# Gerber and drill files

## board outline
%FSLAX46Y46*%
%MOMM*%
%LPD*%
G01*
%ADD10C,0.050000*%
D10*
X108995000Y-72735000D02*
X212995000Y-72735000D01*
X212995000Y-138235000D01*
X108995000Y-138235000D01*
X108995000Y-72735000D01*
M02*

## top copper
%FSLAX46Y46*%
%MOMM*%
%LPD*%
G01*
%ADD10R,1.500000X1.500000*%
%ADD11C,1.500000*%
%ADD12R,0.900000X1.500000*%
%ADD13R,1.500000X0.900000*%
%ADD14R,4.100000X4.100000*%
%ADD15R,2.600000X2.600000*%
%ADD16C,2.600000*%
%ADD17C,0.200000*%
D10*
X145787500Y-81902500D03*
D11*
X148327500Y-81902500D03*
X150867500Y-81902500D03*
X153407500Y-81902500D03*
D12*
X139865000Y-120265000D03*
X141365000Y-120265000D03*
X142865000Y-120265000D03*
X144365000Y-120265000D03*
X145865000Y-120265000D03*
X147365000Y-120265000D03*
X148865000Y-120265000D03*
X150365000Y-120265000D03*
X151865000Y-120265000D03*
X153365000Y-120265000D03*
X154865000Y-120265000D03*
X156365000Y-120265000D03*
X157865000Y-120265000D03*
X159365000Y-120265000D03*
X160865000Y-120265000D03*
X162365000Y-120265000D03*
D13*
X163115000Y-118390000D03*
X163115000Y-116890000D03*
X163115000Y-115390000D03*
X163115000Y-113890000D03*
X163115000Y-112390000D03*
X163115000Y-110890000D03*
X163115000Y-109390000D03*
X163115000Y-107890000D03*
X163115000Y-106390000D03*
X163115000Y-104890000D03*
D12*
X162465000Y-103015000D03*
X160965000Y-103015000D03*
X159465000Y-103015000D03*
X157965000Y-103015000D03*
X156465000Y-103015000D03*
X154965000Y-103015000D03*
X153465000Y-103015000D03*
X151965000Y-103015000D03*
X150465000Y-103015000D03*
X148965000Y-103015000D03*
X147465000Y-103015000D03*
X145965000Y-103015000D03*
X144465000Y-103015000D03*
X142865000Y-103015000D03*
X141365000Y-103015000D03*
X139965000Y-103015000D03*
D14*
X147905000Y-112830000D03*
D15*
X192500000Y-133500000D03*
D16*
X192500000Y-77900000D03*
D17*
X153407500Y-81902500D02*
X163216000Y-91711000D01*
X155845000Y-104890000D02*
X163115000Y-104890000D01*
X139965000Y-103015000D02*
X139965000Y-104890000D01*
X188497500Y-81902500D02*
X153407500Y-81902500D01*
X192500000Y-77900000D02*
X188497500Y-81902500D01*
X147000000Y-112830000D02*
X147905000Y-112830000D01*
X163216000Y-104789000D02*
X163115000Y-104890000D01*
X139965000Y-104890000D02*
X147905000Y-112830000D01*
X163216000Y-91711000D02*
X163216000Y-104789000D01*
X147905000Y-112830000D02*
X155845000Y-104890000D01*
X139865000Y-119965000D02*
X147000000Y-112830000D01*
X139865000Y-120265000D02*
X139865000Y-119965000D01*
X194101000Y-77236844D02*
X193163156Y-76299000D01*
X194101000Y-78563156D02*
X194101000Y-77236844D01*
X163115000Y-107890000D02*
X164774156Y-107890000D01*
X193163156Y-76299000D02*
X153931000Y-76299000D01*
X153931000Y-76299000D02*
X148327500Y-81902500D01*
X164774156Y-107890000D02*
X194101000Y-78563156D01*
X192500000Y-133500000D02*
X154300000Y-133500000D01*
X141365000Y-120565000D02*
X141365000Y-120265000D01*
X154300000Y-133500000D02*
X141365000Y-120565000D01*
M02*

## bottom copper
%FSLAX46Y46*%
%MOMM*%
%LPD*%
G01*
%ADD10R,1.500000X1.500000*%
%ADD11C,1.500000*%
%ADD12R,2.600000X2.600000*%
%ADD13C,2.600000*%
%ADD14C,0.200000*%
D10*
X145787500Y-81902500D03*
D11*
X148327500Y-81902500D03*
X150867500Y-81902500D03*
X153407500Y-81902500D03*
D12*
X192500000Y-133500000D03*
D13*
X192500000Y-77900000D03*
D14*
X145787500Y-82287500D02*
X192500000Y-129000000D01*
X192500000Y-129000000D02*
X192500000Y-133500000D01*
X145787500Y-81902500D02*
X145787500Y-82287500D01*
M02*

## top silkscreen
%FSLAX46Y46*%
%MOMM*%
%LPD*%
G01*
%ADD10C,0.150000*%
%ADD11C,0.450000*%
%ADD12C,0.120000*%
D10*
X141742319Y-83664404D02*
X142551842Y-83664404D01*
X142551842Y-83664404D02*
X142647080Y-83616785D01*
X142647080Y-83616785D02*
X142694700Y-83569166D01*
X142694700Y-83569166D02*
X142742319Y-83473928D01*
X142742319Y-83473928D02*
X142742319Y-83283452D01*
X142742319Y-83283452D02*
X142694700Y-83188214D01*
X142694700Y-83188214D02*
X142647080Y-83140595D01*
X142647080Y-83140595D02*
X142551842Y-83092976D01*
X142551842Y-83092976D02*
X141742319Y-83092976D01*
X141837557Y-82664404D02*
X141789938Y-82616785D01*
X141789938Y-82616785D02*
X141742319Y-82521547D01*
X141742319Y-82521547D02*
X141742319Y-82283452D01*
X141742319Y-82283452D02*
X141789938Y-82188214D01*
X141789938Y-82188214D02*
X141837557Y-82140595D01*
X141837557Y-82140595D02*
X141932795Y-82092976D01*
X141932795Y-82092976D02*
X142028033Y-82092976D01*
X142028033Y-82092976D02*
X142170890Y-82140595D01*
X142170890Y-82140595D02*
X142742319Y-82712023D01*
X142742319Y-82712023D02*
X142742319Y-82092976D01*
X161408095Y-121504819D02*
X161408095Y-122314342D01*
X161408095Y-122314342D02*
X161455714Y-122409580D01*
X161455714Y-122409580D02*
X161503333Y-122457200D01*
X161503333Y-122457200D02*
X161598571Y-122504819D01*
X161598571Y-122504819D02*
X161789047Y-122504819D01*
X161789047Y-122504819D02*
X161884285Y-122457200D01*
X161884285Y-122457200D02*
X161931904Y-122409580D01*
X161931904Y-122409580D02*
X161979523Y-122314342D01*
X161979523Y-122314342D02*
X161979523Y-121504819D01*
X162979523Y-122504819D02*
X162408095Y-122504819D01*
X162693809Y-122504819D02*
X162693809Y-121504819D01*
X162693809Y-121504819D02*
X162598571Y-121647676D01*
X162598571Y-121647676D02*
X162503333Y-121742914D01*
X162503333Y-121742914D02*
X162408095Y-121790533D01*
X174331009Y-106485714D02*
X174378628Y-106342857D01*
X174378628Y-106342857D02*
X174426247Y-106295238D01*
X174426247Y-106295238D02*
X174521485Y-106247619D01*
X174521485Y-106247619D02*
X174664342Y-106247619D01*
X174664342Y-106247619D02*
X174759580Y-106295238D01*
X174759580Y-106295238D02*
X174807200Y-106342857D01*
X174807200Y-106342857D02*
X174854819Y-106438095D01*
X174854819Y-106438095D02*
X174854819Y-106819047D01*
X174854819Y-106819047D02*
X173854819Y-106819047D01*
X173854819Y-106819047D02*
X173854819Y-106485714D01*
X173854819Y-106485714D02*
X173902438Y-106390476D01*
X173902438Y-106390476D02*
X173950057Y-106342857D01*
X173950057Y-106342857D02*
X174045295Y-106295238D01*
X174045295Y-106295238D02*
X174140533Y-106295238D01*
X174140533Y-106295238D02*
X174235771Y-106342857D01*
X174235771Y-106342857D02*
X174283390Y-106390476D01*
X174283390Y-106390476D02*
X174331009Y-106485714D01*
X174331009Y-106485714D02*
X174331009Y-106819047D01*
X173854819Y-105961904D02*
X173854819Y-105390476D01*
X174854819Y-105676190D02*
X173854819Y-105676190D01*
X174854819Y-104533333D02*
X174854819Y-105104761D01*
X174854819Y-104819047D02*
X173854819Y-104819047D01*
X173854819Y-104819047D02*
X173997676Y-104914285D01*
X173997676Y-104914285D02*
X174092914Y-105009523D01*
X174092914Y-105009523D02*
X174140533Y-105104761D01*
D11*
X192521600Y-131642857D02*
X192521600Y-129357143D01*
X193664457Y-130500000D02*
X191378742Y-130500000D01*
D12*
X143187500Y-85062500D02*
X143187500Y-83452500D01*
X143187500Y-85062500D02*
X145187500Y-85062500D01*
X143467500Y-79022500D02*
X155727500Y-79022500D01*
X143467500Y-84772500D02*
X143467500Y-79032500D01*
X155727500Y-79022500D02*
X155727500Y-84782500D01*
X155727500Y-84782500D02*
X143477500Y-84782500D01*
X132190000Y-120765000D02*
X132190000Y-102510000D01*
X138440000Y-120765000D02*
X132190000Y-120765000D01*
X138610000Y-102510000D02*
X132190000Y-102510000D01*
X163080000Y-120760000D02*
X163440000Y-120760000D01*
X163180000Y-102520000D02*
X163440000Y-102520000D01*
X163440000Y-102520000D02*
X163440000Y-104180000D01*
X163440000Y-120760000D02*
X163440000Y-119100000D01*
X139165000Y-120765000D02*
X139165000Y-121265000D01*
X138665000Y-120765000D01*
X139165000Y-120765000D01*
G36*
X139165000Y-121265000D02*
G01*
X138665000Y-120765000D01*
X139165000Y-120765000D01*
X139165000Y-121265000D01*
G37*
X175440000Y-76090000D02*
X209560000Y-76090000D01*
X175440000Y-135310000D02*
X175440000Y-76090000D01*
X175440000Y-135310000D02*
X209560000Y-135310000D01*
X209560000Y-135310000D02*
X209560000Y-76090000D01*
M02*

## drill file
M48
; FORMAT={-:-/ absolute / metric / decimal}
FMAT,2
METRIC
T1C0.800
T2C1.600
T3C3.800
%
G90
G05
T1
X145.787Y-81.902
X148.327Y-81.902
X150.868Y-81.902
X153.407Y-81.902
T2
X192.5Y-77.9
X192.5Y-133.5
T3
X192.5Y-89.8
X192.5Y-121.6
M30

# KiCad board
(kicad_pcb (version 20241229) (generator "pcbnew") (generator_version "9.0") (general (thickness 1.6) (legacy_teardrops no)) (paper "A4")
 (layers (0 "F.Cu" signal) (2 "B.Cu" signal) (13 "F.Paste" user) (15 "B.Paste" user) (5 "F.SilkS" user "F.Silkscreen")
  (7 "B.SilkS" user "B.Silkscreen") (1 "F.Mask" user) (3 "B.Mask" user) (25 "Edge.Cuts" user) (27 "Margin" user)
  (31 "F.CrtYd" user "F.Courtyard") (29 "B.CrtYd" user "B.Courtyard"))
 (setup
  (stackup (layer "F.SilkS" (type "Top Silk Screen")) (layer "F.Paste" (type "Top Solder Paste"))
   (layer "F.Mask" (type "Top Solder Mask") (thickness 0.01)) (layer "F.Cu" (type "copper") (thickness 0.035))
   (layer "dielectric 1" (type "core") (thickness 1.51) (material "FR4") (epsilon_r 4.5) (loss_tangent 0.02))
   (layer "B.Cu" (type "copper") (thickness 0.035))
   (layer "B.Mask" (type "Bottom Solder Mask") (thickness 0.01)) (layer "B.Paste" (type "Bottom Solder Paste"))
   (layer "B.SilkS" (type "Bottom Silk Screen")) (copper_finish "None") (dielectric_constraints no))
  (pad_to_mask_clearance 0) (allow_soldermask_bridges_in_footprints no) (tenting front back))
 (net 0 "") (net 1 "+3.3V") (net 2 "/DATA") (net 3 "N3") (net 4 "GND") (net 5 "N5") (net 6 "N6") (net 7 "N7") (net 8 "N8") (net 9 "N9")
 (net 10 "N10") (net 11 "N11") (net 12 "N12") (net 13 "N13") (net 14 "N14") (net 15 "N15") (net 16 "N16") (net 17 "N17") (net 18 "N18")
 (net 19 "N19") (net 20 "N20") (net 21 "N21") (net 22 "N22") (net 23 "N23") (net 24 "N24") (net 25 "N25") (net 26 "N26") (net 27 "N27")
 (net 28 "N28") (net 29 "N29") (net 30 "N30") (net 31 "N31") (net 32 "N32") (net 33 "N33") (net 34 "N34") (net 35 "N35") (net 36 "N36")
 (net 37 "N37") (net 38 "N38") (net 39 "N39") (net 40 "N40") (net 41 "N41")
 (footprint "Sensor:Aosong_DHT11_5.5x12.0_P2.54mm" (layer "F.Cu") (at 145.7875 81.9025 90)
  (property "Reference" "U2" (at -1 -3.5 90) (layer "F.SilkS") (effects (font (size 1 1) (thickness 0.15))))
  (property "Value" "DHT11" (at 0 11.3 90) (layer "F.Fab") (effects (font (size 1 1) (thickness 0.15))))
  (fp_line (start -3.16 -2.6) (end -1.55 -2.6) (stroke (width 0.12) (type solid)) (layer "F.SilkS"))
  (fp_line (start -3.16 -2.6) (end -3.16 -0.6) (stroke (width 0.12) (type solid)) (layer "F.SilkS"))
  (fp_line (start 2.88 -2.32) (end 2.88 9.94) (stroke (width 0.12) (type solid)) (layer "F.SilkS"))
  (fp_line (start -2.87 -2.32) (end 2.87 -2.32) (stroke (width 0.12) (type solid)) (layer "F.SilkS"))
  (fp_line (start 2.88 9.94) (end -2.88 9.94) (stroke (width 0.12) (type solid)) (layer "F.SilkS"))
  (fp_line (start -2.88 9.94) (end -2.88 -2.31) (stroke (width 0.12) (type solid)) (layer "F.SilkS"))
  (pad "1" thru_hole rect (at 0 0 90) (size 1.5 1.5) (drill 0.8) (layers "*.Cu" "*.Mask") (remove_unused_layers no) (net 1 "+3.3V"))
  (pad "2" thru_hole circle (at 0 2.54 90) (size 1.5 1.5) (drill 0.8) (layers "*.Cu" "*.Mask") (remove_unused_layers no) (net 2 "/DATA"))
  (pad "3" thru_hole circle (at 0 5.08 90) (size 1.5 1.5) (drill 0.8) (layers "*.Cu" "*.Mask") (remove_unused_layers no) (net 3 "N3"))
  (pad "4" thru_hole circle (at 0 7.62 90) (size 1.5 1.5) (drill 0.8) (layers "*.Cu" "*.Mask") (remove_unused_layers no) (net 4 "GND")))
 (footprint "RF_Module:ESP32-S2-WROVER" (layer "F.Cu") (at 151.64 111.64 90)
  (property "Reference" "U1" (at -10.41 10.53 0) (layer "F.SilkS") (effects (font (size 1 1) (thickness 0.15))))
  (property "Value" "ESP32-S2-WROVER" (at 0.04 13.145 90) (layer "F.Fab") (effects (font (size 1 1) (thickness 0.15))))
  (fp_line (start -9.125 -19.45) (end 9.13 -19.45) (stroke (width 0.12) (type solid)) (layer "F.SilkS"))
  (fp_line (start -9.125 -13.2) (end -9.125 -19.45) (stroke (width 0.12) (type solid)) (layer "F.SilkS"))
  (fp_line (start 9.13 -13.03) (end 9.13 -19.45) (stroke (width 0.12) (type solid)) (layer "F.SilkS"))
  (fp_line (start -9.12 11.44) (end -9.12 11.8) (stroke (width 0.12) (type solid)) (layer "F.SilkS"))
  (fp_line (start 9.12 11.54) (end 9.12 11.8) (stroke (width 0.12) (type solid)) (layer "F.SilkS"))
  (fp_line (start 9.12 11.8) (end 7.46 11.8) (stroke (width 0.12) (type solid)) (layer "F.SilkS"))
  (fp_line (start -9.12 11.8) (end -7.46 11.8) (stroke (width 0.12) (type solid)) (layer "F.SilkS"))
  (fp_poly
   (pts (xy -9.125 -12.475) (xy -9.625 -12.475) (xy -9.125 -12.975) (xy -9.125 -12.475)) (stroke (width 0.12) (type solid)) (fill yes)
   (layer "F.SilkS"))
  (pad "" smd roundrect (at -2.52 -5.065 90) (size 1.07 1.07) (layers "F.Paste") (roundrect_rratio 0.233645))
  (pad "" smd roundrect (at -2.52 -3.735 90) (size 1.07 1.07) (layers "F.Paste") (roundrect_rratio 0.233645))
  (pad "" smd roundrect (at -2.52 -2.405 90) (size 1.07 1.07) (layers "F.Paste") (roundrect_rratio 0.233645))
  (pad "" smd roundrect (at -1.19 -5.065 90) (size 1.07 1.07) (layers "F.Paste") (roundrect_rratio 0.233645))
  (pad "" smd roundrect (at -1.19 -3.735 90) (size 1.07 1.07) (layers "F.Paste") (roundrect_rratio 0.233645))
  (pad "" smd roundrect (at -1.19 -2.405 90) (size 1.07 1.07) (layers "F.Paste") (roundrect_rratio 0.233645))
  (pad "" smd roundrect (at 0.14 -5.065 90) (size 1.07 1.07) (layers "F.Paste") (roundrect_rratio 0.233645))
  (pad "" smd roundrect (at 0.14 -3.735 90) (size 1.07 1.07) (layers "F.Paste") (roundrect_rratio 0.233645))
  (pad "" smd roundrect (at 0.14 -2.405 90) (size 1.07 1.07) (layers "F.Paste") (roundrect_rratio 0.233645))
  (pad "1" smd rect (at -8.625 -11.775 90) (size 1.5 0.9) (layers "F.Cu" "F.Mask" "F.Paste") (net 4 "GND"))
  (pad "2" smd rect (at -8.625 -10.275 90) (size 1.5 0.9) (layers "F.Cu" "F.Mask" "F.Paste") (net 1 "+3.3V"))
  (pad "3" smd rect (at -8.625 -8.775 90) (size 1.5 0.9) (layers "F.Cu" "F.Mask" "F.Paste") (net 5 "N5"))
  (pad "4" smd rect (at -8.625 -7.275 90) (size 1.5 0.9) (layers "F.Cu" "F.Mask" "F.Paste") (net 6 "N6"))
  (pad "5" smd rect (at -8.625 -5.775 90) (size 1.5 0.9) (layers "F.Cu" "F.Mask" "F.Paste") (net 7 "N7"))
  (pad "6" smd rect (at -8.625 -4.275 90) (size 1.5 0.9) (layers "F.Cu" "F.Mask" "F.Paste") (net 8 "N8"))
  (pad "7" smd rect (at -8.625 -2.775 90) (size 1.5 0.9) (layers "F.Cu" "F.Mask" "F.Paste") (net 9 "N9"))
  (pad "8" smd rect (at -8.625 -1.275 90) (size 1.5 0.9) (layers "F.Cu" "F.Mask" "F.Paste") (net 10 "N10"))
  (pad "9" smd rect (at -8.625 0.225 90) (size 1.5 0.9) (layers "F.Cu" "F.Mask" "F.Paste") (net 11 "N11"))
  (pad "10" smd rect (at -8.625 1.725 90) (size 1.5 0.9) (layers "F.Cu" "F.Mask" "F.Paste") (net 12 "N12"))
  (pad "11" smd rect (at -8.625 3.225 90) (size 1.5 0.9) (layers "F.Cu" "F.Mask" "F.Paste") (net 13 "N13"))
  (pad "12" smd rect (at -8.625 4.725 90) (size 1.5 0.9) (layers "F.Cu" "F.Mask" "F.Paste") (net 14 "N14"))
  (pad "13" smd rect (at -8.625 6.225 90) (size 1.5 0.9) (layers "F.Cu" "F.Mask" "F.Paste") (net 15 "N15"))
  (pad "14" smd rect (at -8.625 7.725 90) (size 1.5 0.9) (layers "F.Cu" "F.Mask" "F.Paste") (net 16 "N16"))
  (pad "15" smd rect (at -8.625 9.225 270) (size 1.5 0.9) (layers "F.Cu" "F.Mask" "F.Paste") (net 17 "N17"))
  (pad "16" smd rect (at -8.625 10.725 270) (size 1.5 0.9) (layers "F.Cu" "F.Mask" "F.Paste") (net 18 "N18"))
  (pad "17" smd rect (at -6.75 11.475 90) (size 0.9 1.5) (layers "F.Cu" "F.Mask" "F.Paste") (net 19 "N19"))
  (pad "18" smd rect (at -5.25 11.475 90) (size 0.9 1.5) (layers "F.Cu" "F.Mask" "F.Paste") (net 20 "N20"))
  (pad "19" smd rect (at -3.75 11.475 90) (size 0.9 1.5) (layers "F.Cu" "F.Mask" "F.Paste") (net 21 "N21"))
  (pad "20" smd rect (at -2.25 11.475 90) (size 0.9 1.5) (layers "F.Cu" "F.Mask" "F.Paste") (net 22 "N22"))
  (pad "21" smd rect (at -0.75 11.475 90) (size 0.9 1.5) (layers "F.Cu" "F.Mask" "F.Paste") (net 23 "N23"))
  (pad "22" smd rect (at 0.75 11.475 90) (size 0.9 1.5) (layers "F.Cu" "F.Mask" "F.Paste") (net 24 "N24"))
  (pad "23" smd rect (at 2.25 11.475 90) (size 0.9 1.5) (layers "F.Cu" "F.Mask" "F.Paste") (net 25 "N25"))
  (pad "24" smd rect (at 3.75 11.475 90) (size 0.9 1.5) (layers "F.Cu" "F.Mask" "F.Paste") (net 2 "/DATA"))
  (pad "25" smd rect (at 5.25 11.475 90) (size 0.9 1.5) (layers "F.Cu" "F.Mask" "F.Paste") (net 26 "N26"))
  (pad "26" smd rect (at 6.75 11.475 90) (size 0.9 1.5) (layers "F.Cu" "F.Mask" "F.Paste") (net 4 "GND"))
  (pad "27" smd rect (at 8.625 10.825 90) (size 1.5 0.9) (layers "F.Cu" "F.Mask" "F.Paste") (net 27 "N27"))
  (pad "28" smd rect (at 8.625 9.325 90) (size 1.5 0.9) (layers "F.Cu" "F.Mask" "F.Paste") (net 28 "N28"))
  (pad "29" smd rect (at 8.625 7.825 90) (size 1.5 0.9) (layers "F.Cu" "F.Mask" "F.Paste") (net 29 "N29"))
  (pad "30" smd rect (at 8.625 6.325 90) (size 1.5 0.9) (layers "F.Cu" "F.Mask" "F.Paste") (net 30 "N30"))
  (pad "31" smd rect (at 8.625 4.825 90) (size 1.5 0.9) (layers "F.Cu" "F.Mask" "F.Paste") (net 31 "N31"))
  (pad "32" smd rect (at 8.625 3.325 90) (size 1.5 0.9) (layers "F.Cu" "F.Mask" "F.Paste") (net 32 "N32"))
  (pad "33" smd rect (at 8.625 1.825 90) (size 1.5 0.9) (layers "F.Cu" "F.Mask" "F.Paste") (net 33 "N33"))
  (pad "34" smd rect (at 8.625 0.325 90) (size 1.5 0.9) (layers "F.Cu" "F.Mask" "F.Paste") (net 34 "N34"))
  (pad "35" smd rect (at 8.625 -1.175 90) (size 1.5 0.9) (layers "F.Cu" "F.Mask" "F.Paste") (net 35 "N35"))
  (pad "36" smd rect (at 8.625 -2.675 90) (size 1.5 0.9) (layers "F.Cu" "F.Mask" "F.Paste") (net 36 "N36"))
  (pad "37" smd rect (at 8.625 -4.175 90) (size 1.5 0.9) (layers "F.Cu" "F.Mask" "F.Paste") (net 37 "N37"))
  (pad "38" smd rect (at 8.625 -5.675 90) (size 1.5 0.9) (layers "F.Cu" "F.Mask" "F.Paste") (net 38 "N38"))
  (pad "39" smd rect (at 8.625 -7.175 90) (size 1.5 0.9) (layers "F.Cu" "F.Mask" "F.Paste") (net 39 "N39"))
  (pad "40" smd rect (at 8.625 -8.775 90) (size 1.5 0.9) (layers "F.Cu" "F.Mask" "F.Paste") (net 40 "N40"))
  (pad "41" smd rect (at 8.625 -10.275 90) (size 1.5 0.9) (layers "F.Cu" "F.Mask" "F.Paste") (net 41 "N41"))
  (pad "42" smd rect (at 8.625 -11.675 90) (size 1.5 0.9) (layers "F.Cu" "F.Mask" "F.Paste") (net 4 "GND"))
  (pad "43" smd rect (at -1.19 -3.735 90) (size 4.1 4.1) (layers "F.Cu" "F.Mask") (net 4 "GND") (zone_connect 2))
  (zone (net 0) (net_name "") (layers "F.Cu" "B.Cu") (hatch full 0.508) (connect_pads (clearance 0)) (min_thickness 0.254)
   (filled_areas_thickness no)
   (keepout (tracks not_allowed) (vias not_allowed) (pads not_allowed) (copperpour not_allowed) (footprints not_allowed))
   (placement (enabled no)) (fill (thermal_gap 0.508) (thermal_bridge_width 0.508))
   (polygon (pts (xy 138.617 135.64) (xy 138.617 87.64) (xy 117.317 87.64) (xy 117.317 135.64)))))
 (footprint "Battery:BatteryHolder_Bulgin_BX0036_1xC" (layer "F.Cu") (at 192.5 133.5 90)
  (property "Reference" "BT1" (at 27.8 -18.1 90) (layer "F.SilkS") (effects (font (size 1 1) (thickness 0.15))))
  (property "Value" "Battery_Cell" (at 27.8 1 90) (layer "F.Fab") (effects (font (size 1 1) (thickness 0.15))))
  (fp_line (start 57.41 -17.06) (end 57.41 17.06) (stroke (width 0.12) (type solid)) (layer "F.SilkS"))
  (fp_line (start -1.81 -17.06) (end 57.41 -17.06) (stroke (width 0.12) (type solid)) (layer "F.SilkS"))
  (fp_line (start -1.81 -17.06) (end -1.81 17.06) (stroke (width 0.12) (type solid)) (layer "F.SilkS"))
  (fp_line (start -1.81 17.06) (end 57.41 17.06) (stroke (width 0.12) (type solid)) (layer "F.SilkS"))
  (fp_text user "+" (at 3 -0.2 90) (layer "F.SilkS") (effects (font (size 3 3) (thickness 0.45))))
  (pad "" np_thru_hole circle (at 11.9 0 90) (size 3.8 3.8) (drill 3.8) (layers "*.Cu" "*.Mask"))
  (pad "" np_thru_hole circle (at 43.7 0 90) (size 3.8 3.8) (drill 3.8) (layers "*.Cu" "*.Mask"))
  (pad "1" thru_hole rect (at 0 0 90) (size 2.6 2.6) (drill 1.6) (layers "*.Cu" "*.Mask") (remove_unused_layers no) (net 1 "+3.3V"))
  (pad "2" thru_hole circle (at 55.6 0 90) (size 2.6 2.6) (drill 1.6) (layers "*.Cu" "*.Mask") (remove_unused_layers no) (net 4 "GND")))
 (gr_rect (start 108.995 72.735) (end 212.995 138.235) (stroke (width 0.05) (type default)) (fill no) (layer "Edge.Cuts"))
 (segment (start 153.4075 81.9025) (end 163.216 91.711) (width 0.2) (layer "F.Cu") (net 4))
 (segment (start 155.845 104.89) (end 163.115 104.89) (width 0.2) (layer "F.Cu") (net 4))
 (segment (start 139.965 103.015) (end 139.965 104.89) (width 0.2) (layer "F.Cu") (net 4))
 (segment (start 188.4975 81.9025) (end 153.4075 81.9025) (width 0.2) (layer "F.Cu") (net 4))
 (segment (start 192.5 77.9) (end 188.4975 81.9025) (width 0.2) (layer "F.Cu") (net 4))
 (segment (start 147 112.83) (end 147.905 112.83) (width 0.2) (layer "F.Cu") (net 4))
 (segment (start 163.216 104.789) (end 163.115 104.89) (width 0.2) (layer "F.Cu") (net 4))
 (segment (start 139.965 104.89) (end 147.905 112.83) (width 0.2) (layer "F.Cu") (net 4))
 (segment (start 163.216 91.711) (end 163.216 104.789) (width 0.2) (layer "F.Cu") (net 4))
 (segment (start 147.905 112.83) (end 155.845 104.89) (width 0.2) (layer "F.Cu") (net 4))
 (segment (start 139.865 119.965) (end 147 112.83) (width 0.2) (layer "F.Cu") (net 4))
 (segment (start 139.865 120.265) (end 139.865 119.965) (width 0.2) (layer "F.Cu") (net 4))
 (segment (start 194.101 77.236844) (end 193.163156 76.299) (width 0.2) (layer "F.Cu") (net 2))
 (segment (start 194.101 78.563156) (end 194.101 77.236844) (width 0.2) (layer "F.Cu") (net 2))
 (segment (start 163.115 107.89) (end 164.774156 107.89) (width 0.2) (layer "F.Cu") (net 2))
 (segment (start 193.163156 76.299) (end 153.931 76.299) (width 0.2) (layer "F.Cu") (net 2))
 (segment (start 153.931 76.299) (end 148.3275 81.9025) (width 0.2) (layer "F.Cu") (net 2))
 (segment (start 164.774156 107.89) (end 194.101 78.563156) (width 0.2) (layer "F.Cu") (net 2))
 (segment (start 192.5 133.5) (end 154.3 133.5) (width 0.2) (layer "F.Cu") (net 1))
 (segment (start 141.365 120.565) (end 141.365 120.265) (width 0.2) (layer "F.Cu") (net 1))
 (segment (start 154.3 133.5) (end 141.365 120.565) (width 0.2) (layer "F.Cu") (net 1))
 (segment (start 145.7875 82.2875) (end 192.5 129) (width 0.2) (layer "B.Cu") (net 1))
 (segment (start 192.5 129) (end 192.5 133.5) (width 0.2) (layer "B.Cu") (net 1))
 (segment (start 145.7875 81.9025) (end 145.7875 82.2875) (width 0.2) (layer "B.Cu") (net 1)))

